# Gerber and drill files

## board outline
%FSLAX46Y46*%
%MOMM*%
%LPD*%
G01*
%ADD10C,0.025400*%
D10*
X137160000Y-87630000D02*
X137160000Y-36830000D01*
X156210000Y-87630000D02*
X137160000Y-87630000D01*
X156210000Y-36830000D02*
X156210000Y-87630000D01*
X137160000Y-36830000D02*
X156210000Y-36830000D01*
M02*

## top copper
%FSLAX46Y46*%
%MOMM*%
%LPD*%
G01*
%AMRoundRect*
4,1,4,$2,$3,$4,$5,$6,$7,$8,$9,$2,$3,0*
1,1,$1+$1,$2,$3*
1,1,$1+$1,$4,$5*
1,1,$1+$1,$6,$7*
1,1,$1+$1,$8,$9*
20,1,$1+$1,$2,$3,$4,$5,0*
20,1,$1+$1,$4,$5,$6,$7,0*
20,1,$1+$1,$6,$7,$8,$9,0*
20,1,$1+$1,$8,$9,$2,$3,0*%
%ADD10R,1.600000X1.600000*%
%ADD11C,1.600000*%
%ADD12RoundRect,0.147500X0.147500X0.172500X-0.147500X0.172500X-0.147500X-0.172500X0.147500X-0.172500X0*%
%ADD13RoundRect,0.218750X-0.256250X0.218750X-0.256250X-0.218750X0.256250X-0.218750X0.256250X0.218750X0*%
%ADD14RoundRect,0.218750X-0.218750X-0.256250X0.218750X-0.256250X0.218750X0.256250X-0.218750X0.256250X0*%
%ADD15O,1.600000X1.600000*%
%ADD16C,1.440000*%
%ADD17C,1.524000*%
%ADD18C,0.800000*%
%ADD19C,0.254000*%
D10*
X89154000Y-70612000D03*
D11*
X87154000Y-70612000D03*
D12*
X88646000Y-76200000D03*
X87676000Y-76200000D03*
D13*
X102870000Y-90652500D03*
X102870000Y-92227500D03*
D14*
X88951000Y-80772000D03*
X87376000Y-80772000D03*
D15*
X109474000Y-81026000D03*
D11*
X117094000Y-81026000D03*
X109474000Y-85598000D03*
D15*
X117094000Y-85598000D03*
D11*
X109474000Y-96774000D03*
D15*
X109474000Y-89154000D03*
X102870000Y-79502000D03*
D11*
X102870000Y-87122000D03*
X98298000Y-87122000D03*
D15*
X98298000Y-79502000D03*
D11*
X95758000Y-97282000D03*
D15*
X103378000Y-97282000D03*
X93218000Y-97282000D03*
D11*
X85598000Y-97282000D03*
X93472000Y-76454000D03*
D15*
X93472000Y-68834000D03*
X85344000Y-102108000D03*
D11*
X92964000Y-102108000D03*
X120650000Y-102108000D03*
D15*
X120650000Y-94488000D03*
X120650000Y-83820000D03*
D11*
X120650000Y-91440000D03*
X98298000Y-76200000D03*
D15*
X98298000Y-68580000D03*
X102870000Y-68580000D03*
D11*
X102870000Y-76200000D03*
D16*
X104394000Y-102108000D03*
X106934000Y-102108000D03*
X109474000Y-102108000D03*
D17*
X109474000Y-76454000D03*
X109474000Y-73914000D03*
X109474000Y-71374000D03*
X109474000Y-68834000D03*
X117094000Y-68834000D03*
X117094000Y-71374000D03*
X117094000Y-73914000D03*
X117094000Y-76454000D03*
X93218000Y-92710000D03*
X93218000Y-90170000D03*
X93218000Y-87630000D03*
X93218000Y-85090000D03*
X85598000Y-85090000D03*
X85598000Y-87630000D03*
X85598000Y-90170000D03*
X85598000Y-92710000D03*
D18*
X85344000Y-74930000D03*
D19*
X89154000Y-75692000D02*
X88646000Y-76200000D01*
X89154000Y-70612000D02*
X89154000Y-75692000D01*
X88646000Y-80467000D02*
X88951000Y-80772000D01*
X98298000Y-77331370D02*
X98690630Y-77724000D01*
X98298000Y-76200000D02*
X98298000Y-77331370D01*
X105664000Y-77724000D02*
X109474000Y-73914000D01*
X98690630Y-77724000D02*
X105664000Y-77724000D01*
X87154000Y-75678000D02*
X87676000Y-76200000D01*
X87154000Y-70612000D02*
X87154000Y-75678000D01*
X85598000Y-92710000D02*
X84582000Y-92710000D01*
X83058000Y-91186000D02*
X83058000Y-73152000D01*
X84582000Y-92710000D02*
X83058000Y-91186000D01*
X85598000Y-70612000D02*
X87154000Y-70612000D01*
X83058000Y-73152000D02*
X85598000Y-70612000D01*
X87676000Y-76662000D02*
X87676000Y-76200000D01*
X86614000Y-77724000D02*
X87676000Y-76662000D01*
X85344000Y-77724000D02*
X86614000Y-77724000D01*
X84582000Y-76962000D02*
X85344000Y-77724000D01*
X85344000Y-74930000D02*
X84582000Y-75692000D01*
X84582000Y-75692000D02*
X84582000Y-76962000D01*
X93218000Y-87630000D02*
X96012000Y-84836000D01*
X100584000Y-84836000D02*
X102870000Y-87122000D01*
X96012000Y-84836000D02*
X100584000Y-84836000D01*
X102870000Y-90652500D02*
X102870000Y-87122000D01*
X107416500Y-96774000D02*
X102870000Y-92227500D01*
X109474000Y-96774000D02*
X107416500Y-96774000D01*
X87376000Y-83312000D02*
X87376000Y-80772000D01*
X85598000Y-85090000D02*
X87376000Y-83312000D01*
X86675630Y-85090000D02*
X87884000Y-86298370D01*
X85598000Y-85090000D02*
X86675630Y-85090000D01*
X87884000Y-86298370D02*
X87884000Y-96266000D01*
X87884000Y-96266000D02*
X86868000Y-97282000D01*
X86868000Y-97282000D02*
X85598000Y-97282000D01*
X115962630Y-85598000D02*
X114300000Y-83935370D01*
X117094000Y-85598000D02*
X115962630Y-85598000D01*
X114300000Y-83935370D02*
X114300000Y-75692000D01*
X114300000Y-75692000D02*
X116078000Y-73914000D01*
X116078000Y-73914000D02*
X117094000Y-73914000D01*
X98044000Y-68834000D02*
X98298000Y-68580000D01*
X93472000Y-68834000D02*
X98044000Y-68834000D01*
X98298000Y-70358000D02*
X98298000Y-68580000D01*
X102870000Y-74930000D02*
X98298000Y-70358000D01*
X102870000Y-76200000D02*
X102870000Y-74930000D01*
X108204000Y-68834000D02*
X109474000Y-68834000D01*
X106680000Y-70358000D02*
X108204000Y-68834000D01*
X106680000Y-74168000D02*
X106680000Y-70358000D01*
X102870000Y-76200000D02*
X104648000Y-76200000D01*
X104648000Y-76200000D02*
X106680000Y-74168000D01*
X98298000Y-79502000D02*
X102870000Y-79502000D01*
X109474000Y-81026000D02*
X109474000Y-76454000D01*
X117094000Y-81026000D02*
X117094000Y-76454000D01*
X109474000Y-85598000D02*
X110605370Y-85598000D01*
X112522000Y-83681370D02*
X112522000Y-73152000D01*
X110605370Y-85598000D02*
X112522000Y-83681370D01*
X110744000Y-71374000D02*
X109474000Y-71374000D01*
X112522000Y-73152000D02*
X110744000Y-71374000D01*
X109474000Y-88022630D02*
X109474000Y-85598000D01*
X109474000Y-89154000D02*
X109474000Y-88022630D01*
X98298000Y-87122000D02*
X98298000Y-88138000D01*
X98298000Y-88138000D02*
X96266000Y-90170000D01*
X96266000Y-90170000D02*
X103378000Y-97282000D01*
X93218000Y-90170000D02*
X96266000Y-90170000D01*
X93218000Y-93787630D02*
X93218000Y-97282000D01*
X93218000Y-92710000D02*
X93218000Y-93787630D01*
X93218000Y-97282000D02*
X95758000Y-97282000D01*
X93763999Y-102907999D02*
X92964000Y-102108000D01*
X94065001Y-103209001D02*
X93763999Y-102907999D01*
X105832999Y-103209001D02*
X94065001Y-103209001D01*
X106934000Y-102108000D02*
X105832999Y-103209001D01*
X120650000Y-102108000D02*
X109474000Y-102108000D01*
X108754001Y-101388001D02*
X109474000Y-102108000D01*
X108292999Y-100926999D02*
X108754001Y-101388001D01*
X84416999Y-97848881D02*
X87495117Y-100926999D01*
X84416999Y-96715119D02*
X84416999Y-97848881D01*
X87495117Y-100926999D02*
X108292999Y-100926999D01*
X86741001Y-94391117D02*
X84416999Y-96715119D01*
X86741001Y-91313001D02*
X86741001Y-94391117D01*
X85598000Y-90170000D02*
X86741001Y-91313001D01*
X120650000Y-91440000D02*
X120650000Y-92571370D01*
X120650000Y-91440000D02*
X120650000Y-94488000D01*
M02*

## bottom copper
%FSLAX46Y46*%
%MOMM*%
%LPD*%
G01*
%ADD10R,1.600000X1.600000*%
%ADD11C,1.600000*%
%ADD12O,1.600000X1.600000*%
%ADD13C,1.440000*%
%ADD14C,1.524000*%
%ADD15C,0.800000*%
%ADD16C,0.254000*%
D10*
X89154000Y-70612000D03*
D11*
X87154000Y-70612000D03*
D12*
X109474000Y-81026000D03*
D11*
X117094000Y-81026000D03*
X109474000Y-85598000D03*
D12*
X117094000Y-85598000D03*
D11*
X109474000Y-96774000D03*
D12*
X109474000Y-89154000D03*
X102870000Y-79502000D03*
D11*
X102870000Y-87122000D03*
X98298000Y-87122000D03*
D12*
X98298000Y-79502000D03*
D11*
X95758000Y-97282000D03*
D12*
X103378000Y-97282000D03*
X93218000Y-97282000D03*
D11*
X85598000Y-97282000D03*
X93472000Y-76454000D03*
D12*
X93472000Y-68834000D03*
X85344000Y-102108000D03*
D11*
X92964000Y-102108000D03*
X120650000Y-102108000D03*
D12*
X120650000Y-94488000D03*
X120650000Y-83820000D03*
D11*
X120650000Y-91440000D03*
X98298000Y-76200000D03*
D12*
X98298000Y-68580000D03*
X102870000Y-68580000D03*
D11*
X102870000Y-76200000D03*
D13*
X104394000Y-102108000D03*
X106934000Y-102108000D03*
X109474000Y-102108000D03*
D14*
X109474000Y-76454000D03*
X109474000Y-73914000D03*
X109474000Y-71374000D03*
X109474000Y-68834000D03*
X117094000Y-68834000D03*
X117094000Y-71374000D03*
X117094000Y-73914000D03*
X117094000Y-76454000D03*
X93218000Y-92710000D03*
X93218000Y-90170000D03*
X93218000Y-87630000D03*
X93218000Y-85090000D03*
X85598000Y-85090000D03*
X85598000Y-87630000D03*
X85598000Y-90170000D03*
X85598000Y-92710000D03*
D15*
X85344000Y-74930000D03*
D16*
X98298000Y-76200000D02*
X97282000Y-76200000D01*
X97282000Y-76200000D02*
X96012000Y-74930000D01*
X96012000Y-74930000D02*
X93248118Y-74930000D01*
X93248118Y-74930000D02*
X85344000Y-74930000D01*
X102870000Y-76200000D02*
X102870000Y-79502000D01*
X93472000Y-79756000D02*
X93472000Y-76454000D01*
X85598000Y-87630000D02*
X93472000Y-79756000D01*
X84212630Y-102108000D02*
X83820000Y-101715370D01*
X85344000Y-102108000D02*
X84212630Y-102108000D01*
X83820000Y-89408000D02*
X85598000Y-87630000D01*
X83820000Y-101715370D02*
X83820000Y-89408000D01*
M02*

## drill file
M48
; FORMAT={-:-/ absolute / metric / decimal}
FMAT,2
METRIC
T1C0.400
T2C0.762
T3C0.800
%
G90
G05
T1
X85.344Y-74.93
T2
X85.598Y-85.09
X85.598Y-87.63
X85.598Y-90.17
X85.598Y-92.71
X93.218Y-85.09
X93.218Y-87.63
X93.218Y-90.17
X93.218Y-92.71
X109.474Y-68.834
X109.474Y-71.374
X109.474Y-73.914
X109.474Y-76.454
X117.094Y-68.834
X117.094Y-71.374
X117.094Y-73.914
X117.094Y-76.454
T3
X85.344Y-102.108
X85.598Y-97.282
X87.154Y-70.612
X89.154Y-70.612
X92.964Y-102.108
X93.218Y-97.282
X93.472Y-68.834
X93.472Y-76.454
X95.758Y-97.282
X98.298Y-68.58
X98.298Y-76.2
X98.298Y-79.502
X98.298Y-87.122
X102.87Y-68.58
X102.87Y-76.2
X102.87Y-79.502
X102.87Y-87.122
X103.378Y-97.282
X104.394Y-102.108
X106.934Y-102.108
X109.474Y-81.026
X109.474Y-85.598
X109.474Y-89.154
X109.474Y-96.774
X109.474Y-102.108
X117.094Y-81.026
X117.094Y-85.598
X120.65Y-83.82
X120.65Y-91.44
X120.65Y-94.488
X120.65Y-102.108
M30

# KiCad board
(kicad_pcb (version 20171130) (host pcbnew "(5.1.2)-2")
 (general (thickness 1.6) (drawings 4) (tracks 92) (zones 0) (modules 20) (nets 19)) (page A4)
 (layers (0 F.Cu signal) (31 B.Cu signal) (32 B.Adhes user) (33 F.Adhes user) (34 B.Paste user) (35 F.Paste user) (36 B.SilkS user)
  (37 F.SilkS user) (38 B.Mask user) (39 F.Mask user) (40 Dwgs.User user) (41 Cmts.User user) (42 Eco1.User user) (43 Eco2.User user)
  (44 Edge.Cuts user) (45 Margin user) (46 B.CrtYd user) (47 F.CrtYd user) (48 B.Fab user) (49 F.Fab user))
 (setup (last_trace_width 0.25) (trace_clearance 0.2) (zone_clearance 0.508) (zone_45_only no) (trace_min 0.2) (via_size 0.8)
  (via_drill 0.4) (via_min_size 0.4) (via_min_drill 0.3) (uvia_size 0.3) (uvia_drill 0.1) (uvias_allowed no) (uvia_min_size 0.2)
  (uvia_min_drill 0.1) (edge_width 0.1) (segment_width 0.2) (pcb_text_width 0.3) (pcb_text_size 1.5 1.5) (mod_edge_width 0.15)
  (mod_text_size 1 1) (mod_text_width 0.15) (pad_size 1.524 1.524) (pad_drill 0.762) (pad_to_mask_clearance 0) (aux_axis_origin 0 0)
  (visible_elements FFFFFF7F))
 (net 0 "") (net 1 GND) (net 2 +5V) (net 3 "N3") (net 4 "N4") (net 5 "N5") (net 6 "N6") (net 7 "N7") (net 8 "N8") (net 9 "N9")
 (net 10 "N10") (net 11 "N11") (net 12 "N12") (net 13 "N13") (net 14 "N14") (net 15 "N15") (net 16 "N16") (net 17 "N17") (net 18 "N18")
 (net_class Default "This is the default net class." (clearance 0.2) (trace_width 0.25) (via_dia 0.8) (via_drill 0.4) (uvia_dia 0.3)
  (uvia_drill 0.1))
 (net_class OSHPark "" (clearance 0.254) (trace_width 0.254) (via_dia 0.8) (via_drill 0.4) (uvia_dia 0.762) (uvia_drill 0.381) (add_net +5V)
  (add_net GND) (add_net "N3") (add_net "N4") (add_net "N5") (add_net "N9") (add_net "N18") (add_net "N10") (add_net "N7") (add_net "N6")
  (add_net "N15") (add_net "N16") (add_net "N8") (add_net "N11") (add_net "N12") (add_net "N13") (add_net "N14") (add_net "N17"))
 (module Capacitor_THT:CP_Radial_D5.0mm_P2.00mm (layer F.Cu) (at 89.154 70.612 180)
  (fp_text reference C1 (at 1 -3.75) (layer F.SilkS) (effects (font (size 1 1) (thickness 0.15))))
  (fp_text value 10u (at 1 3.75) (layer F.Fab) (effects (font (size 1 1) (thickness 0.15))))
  (pad 1 thru_hole rect (at 0 0 180) (size 1.6 1.6) (drill 0.8) (layers *.Cu *.Mask) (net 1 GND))
  (pad 2 thru_hole circle (at 2 0 180) (size 1.6 1.6) (drill 0.8) (layers *.Cu *.Mask) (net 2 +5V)))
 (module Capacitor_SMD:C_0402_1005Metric (layer F.Cu) (at 88.161 76.2 180)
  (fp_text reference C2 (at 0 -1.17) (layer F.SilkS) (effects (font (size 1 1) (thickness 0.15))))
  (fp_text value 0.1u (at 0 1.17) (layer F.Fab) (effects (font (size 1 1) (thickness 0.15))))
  (pad 1 smd roundrect (at -0.485 0 180) (size 0.59 0.64) (layers F.Cu F.Paste F.Mask) (roundrect_rratio 0.25) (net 1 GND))
  (pad 2 smd roundrect (at 0.485 0 180) (size 0.59 0.64) (layers F.Cu F.Paste F.Mask) (roundrect_rratio 0.25) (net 2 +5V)))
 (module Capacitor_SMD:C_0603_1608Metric (layer F.Cu) (at 102.87 91.44 270)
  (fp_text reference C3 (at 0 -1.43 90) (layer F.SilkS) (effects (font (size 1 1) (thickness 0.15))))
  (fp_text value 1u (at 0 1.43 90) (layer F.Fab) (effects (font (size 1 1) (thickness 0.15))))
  (pad 1 smd roundrect (at -0.7875 0 270) (size 0.875 0.95) (layers F.Cu F.Paste F.Mask) (roundrect_rratio 0.25) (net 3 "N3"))
  (pad 2 smd roundrect (at 0.7875 0 270) (size 0.875 0.95) (layers F.Cu F.Paste F.Mask) (roundrect_rratio 0.25) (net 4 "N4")))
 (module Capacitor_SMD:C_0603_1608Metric (layer F.Cu) (at 88.1635 80.772)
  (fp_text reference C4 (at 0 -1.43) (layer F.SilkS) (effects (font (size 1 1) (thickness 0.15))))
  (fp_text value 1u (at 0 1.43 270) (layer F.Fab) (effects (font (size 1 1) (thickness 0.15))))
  (pad 2 smd roundrect (at 0.7875 0) (size 0.875 0.95) (layers F.Cu F.Paste F.Mask) (roundrect_rratio 0.25) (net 1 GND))
  (pad 1 smd roundrect (at -0.7875 0) (size 0.875 0.95) (layers F.Cu F.Paste F.Mask) (roundrect_rratio 0.25) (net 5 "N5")))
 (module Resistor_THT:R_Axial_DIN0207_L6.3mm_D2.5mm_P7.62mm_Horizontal (layer F.Cu) (at 117.094 81.026 180)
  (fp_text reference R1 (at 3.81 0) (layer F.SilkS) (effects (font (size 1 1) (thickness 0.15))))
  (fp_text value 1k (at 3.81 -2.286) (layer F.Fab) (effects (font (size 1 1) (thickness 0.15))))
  (pad 2 thru_hole oval (at 7.62 0 180) (size 1.6 1.6) (drill 0.8) (layers *.Cu *.Mask) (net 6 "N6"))
  (pad 1 thru_hole circle (at 0 0 180) (size 1.6 1.6) (drill 0.8) (layers *.Cu *.Mask) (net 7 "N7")))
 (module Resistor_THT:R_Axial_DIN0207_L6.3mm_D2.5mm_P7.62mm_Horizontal (layer F.Cu) (at 109.474 85.598)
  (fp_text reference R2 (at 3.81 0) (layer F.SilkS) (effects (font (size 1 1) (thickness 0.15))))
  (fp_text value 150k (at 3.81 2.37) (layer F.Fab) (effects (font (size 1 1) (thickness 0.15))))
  (pad 1 thru_hole circle (at 0 0) (size 1.6 1.6) (drill 0.8) (layers *.Cu *.Mask) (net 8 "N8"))
  (pad 2 thru_hole oval (at 7.62 0) (size 1.6 1.6) (drill 0.8) (layers *.Cu *.Mask) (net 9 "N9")))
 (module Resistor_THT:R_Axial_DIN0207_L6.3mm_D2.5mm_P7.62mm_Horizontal (layer F.Cu) (at 109.474 96.774 90)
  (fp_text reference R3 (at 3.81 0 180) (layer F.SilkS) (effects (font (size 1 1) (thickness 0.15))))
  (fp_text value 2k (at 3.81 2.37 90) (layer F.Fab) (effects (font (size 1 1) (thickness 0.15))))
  (pad 1 thru_hole circle (at 0 0 90) (size 1.6 1.6) (drill 0.8) (layers *.Cu *.Mask) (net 4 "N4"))
  (pad 2 thru_hole oval (at 7.62 0 90) (size 1.6 1.6) (drill 0.8) (layers *.Cu *.Mask) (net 8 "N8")))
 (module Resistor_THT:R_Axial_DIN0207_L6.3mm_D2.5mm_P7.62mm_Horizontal (layer F.Cu) (at 102.87 87.122 90)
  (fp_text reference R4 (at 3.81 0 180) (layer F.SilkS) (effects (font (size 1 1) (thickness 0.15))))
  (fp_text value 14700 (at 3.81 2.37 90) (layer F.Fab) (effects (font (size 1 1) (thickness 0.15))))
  (pad 2 thru_hole oval (at 7.62 0 90) (size 1.6 1.6) (drill 0.8) (layers *.Cu *.Mask) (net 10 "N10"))
  (pad 1 thru_hole circle (at 0 0 90) (size 1.6 1.6) (drill 0.8) (layers *.Cu *.Mask) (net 3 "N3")))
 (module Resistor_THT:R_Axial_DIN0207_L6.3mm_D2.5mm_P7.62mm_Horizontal (layer F.Cu) (at 98.298 87.122 90)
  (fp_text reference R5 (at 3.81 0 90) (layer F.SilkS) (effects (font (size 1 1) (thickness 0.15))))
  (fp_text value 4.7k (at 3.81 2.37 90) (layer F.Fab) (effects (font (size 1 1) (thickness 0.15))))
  (pad 1 thru_hole circle (at 0 0 90) (size 1.6 1.6) (drill 0.8) (layers *.Cu *.Mask) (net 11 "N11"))
  (pad 2 thru_hole oval (at 7.62 0 90) (size 1.6 1.6) (drill 0.8) (layers *.Cu *.Mask) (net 10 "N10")))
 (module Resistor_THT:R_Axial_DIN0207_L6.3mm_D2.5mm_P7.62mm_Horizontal (layer F.Cu) (at 95.758 97.282)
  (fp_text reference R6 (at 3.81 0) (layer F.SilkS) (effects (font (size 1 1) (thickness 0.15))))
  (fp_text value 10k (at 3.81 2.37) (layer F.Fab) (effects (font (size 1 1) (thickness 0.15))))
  (pad 1 thru_hole circle (at 0 0) (size 1.6 1.6) (drill 0.8) (layers *.Cu *.Mask) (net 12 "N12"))
  (pad 2 thru_hole oval (at 7.62 0) (size 1.6 1.6) (drill 0.8) (layers *.Cu *.Mask) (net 11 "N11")))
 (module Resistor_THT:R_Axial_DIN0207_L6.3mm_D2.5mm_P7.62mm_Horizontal (layer F.Cu) (at 85.598 97.282)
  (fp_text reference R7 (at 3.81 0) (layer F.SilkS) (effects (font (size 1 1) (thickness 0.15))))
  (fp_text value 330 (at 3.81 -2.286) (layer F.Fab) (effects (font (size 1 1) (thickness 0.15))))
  (pad 2 thru_hole oval (at 7.62 0) (size 1.6 1.6) (drill 0.8) (layers *.Cu *.Mask) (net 12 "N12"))
  (pad 1 thru_hole circle (at 0 0) (size 1.6 1.6) (drill 0.8) (layers *.Cu *.Mask) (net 5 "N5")))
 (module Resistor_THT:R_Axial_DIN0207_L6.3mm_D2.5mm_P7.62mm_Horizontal (layer F.Cu) (at 93.472 76.454 90)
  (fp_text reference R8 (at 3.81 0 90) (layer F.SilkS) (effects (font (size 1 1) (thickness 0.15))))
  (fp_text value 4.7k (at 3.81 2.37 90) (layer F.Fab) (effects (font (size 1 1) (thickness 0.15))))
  (pad 1 thru_hole circle (at 0 0 90) (size 1.6 1.6) (drill 0.8) (layers *.Cu *.Mask) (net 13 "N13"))
  (pad 2 thru_hole oval (at 7.62 0 90) (size 1.6 1.6) (drill 0.8) (layers *.Cu *.Mask) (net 10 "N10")))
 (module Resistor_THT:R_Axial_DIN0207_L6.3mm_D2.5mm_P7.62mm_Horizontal (layer F.Cu) (at 92.964 102.108 180)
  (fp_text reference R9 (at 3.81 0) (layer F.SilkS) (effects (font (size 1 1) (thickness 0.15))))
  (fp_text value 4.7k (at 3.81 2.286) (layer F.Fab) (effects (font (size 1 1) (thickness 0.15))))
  (pad 2 thru_hole oval (at 7.62 0 180) (size 1.6 1.6) (drill 0.8) (layers *.Cu *.Mask) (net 13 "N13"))
  (pad 1 thru_hole circle (at 0 0 180) (size 1.6 1.6) (drill 0.8) (layers *.Cu *.Mask) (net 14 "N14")))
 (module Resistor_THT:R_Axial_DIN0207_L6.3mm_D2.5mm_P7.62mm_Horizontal (layer F.Cu) (at 120.65 102.108 90)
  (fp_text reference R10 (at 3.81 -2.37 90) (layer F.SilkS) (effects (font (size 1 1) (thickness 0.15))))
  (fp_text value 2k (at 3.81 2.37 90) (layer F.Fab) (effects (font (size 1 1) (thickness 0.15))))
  (pad 1 thru_hole circle (at 0 0 90) (size 1.6 1.6) (drill 0.8) (layers *.Cu *.Mask) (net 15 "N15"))
  (pad 2 thru_hole oval (at 7.62 0 90) (size 1.6 1.6) (drill 0.8) (layers *.Cu *.Mask) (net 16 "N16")))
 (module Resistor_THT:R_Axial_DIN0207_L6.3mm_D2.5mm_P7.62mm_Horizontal (layer F.Cu) (at 120.65 91.44 90)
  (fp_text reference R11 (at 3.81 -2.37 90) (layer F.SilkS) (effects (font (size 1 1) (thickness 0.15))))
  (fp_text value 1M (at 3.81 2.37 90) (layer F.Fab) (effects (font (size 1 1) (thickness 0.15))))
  (pad 2 thru_hole oval (at 7.62 0 90) (size 1.6 1.6) (drill 0.8) (layers *.Cu *.Mask) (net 1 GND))
  (pad 1 thru_hole circle (at 0 0 90) (size 1.6 1.6) (drill 0.8) (layers *.Cu *.Mask) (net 16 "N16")))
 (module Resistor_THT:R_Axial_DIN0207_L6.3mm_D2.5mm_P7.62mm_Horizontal (layer F.Cu) (at 98.298 76.2 90)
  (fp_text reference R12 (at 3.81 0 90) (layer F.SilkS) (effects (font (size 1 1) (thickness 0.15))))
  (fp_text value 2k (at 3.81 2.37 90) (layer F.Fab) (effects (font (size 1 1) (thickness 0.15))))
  (pad 1 thru_hole circle (at 0 0 90) (size 1.6 1.6) (drill 0.8) (layers *.Cu *.Mask) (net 2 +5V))
  (pad 2 thru_hole oval (at 7.62 0 90) (size 1.6 1.6) (drill 0.8) (layers *.Cu *.Mask) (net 10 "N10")))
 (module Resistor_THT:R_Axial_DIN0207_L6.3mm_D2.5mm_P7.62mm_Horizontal (layer F.Cu) (at 102.87 76.2 90)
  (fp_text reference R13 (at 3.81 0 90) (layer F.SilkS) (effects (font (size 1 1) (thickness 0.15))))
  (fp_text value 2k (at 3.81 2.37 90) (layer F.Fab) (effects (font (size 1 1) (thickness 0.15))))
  (pad 2 thru_hole oval (at 7.62 0 90) (size 1.6 1.6) (drill 0.8) (layers *.Cu *.Mask) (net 1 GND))
  (pad 1 thru_hole circle (at 0 0 90) (size 1.6 1.6) (drill 0.8) (layers *.Cu *.Mask) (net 10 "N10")))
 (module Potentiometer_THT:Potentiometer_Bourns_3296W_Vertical (layer F.Cu) (at 104.394 102.108 180)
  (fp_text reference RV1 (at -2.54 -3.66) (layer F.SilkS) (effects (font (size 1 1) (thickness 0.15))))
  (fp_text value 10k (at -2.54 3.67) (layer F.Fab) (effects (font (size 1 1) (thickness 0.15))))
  (pad 1 thru_hole circle (at 0 0 180) (size 1.44 1.44) (drill 0.8) (layers *.Cu *.Mask) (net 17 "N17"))
  (pad 2 thru_hole circle (at -2.54 0 180) (size 1.44 1.44) (drill 0.8) (layers *.Cu *.Mask) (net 14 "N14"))
  (pad 3 thru_hole circle (at -5.08 0 180) (size 1.44 1.44) (drill 0.8) (layers *.Cu *.Mask) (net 15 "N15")))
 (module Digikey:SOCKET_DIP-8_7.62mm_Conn (layer F.Cu) (at 117.094 76.454 180)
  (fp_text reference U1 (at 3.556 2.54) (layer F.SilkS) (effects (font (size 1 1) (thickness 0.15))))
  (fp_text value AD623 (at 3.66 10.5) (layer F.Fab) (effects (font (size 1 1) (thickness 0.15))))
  (pad 8 thru_hole circle (at 7.62 0 180) (size 1.524 1.524) (drill 0.762) (layers *.Cu *.Mask) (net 6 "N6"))
  (pad 7 thru_hole circle (at 7.62 2.54 180) (size 1.524 1.524) (drill 0.762) (layers *.Cu *.Mask) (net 2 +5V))
  (pad 6 thru_hole circle (at 7.62 5.08 180) (size 1.524 1.524) (drill 0.762) (layers *.Cu *.Mask) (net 8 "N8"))
  (pad 5 thru_hole circle (at 7.62 7.62 180) (size 1.524 1.524) (drill 0.762) (layers *.Cu *.Mask) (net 10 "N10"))
  (pad 4 thru_hole circle (at 0 7.62 180) (size 1.524 1.524) (drill 0.762) (layers *.Cu *.Mask) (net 1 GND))
  (pad 3 thru_hole circle (at 0 5.08 180) (size 1.524 1.524) (drill 0.762) (layers *.Cu *.Mask) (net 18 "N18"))
  (pad 2 thru_hole circle (at 0 2.54 180) (size 1.524 1.524) (drill 0.762) (layers *.Cu *.Mask) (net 9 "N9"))
  (pad 1 thru_hole circle (at 0 0 180) (size 1.524 1.524) (drill 0.762) (layers *.Cu *.Mask) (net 7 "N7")))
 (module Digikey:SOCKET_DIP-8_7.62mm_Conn (layer F.Cu) (at 93.218 92.71 180)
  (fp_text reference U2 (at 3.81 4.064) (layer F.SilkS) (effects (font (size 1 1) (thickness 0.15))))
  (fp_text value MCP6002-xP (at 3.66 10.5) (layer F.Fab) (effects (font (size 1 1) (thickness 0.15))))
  (pad 1 thru_hole circle (at 0 0 180) (size 1.524 1.524) (drill 0.762) (layers *.Cu *.Mask) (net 12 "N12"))
  (pad 2 thru_hole circle (at 0 2.54 180) (size 1.524 1.524) (drill 0.762) (layers *.Cu *.Mask) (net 11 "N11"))
  (pad 3 thru_hole circle (at 0 5.08 180) (size 1.524 1.524) (drill 0.762) (layers *.Cu *.Mask) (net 3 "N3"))
  (pad 4 thru_hole circle (at 0 7.62 180) (size 1.524 1.524) (drill 0.762) (layers *.Cu *.Mask) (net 1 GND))
  (pad 5 thru_hole circle (at 7.62 7.62 180) (size 1.524 1.524) (drill 0.762) (layers *.Cu *.Mask) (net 5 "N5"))
  (pad 6 thru_hole circle (at 7.62 5.08 180) (size 1.524 1.524) (drill 0.762) (layers *.Cu *.Mask) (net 13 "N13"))
  (pad 7 thru_hole circle (at 7.62 2.54 180) (size 1.524 1.524) (drill 0.762) (layers *.Cu *.Mask) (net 15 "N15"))
  (pad 8 thru_hole circle (at 7.62 0 180) (size 1.524 1.524) (drill 0.762) (layers *.Cu *.Mask) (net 2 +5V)))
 (gr_line (start 137.16 87.63) (end 137.16 36.83) (layer Edge.Cuts) (width 0.0254))
 (gr_line (start 156.21 87.63) (end 137.16 87.63) (layer Edge.Cuts) (width 0.0254))
 (gr_line (start 156.21 36.83) (end 156.21 87.63) (layer Edge.Cuts) (width 0.0254))
 (gr_line (start 137.16 36.83) (end 156.21 36.83) (layer Edge.Cuts) (width 0.0254))
 (segment (start 89.154 75.692) (end 88.646 76.2) (width 0.254) (layer F.Cu) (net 1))
 (segment (start 89.154 70.612) (end 89.154 75.692) (width 0.254) (layer F.Cu) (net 1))
 (segment (start 88.646 80.467) (end 88.951 80.772) (width 0.254) (layer F.Cu) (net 1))
 (segment (start 98.298 77.33137) (end 98.69063 77.724) (width 0.254) (layer F.Cu) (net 2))
 (segment (start 98.298 76.2) (end 98.298 77.33137) (width 0.254) (layer F.Cu) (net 2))
 (segment (start 105.664 77.724) (end 109.474 73.914) (width 0.254) (layer F.Cu) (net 2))
 (segment (start 98.69063 77.724) (end 105.664 77.724) (width 0.254) (layer F.Cu) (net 2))
 (segment (start 87.154 75.678) (end 87.676 76.2) (width 0.254) (layer F.Cu) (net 2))
 (segment (start 87.154 70.612) (end 87.154 75.678) (width 0.254) (layer F.Cu) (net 2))
 (segment (start 85.598 92.71) (end 84.582 92.71) (width 0.254) (layer F.Cu) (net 2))
 (segment (start 83.058 91.186) (end 83.058 73.152) (width 0.254) (layer F.Cu) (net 2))
 (segment (start 84.582 92.71) (end 83.058 91.186) (width 0.254) (layer F.Cu) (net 2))
 (segment (start 85.598 70.612) (end 87.154 70.612) (width 0.254) (layer F.Cu) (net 2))
 (segment (start 83.058 73.152) (end 85.598 70.612) (width 0.254) (layer F.Cu) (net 2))
 (segment (start 98.298 76.2) (end 97.282 76.2) (width 0.254) (layer B.Cu) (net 2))
 (segment (start 97.282 76.2) (end 96.012 74.93) (width 0.254) (layer B.Cu) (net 2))
 (via (at 85.344 74.93) (size 0.8) (drill 0.4) (layers F.Cu B.Cu) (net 2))
 (segment (start 96.012 74.93) (end 93.248118 74.93) (width 0.254) (layer B.Cu) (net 2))
 (segment (start 93.248118 74.93) (end 85.344 74.93) (width 0.254) (layer B.Cu) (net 2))
 (segment (start 87.676 76.662) (end 87.676 76.2) (width 0.254) (layer F.Cu) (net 2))
 (segment (start 86.614 77.724) (end 87.676 76.662) (width 0.254) (layer F.Cu) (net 2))
 (segment (start 85.344 77.724) (end 86.614 77.724) (width 0.254) (layer F.Cu) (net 2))
 (segment (start 84.582 76.962) (end 85.344 77.724) (width 0.254) (layer F.Cu) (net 2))
 (segment (start 85.344 74.93) (end 84.582 75.692) (width 0.254) (layer F.Cu) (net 2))
 (segment (start 84.582 75.692) (end 84.582 76.962) (width 0.254) (layer F.Cu) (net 2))
 (segment (start 93.218 87.63) (end 96.012 84.836) (width 0.254) (layer F.Cu) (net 3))
 (segment (start 100.584 84.836) (end 102.87 87.122) (width 0.254) (layer F.Cu) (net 3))
 (segment (start 96.012 84.836) (end 100.584 84.836) (width 0.254) (layer F.Cu) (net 3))
 (segment (start 102.87 90.6525) (end 102.87 87.122) (width 0.254) (layer F.Cu) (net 3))
 (segment (start 107.4165 96.774) (end 102.87 92.2275) (width 0.254) (layer F.Cu) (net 4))
 (segment (start 109.474 96.774) (end 107.4165 96.774) (width 0.254) (layer F.Cu) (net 4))
 (segment (start 87.376 83.312) (end 87.376 80.772) (width 0.254) (layer F.Cu) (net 5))
 (segment (start 85.598 85.09) (end 87.376 83.312) (width 0.254) (layer F.Cu) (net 5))
 (segment (start 86.67563 85.09) (end 87.884 86.29837) (width 0.254) (layer F.Cu) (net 5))
 (segment (start 85.598 85.09) (end 86.67563 85.09) (width 0.254) (layer F.Cu) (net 5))
 (segment (start 87.884 86.29837) (end 87.884 96.266) (width 0.254) (layer F.Cu) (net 5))
 (segment (start 87.884 96.266) (end 86.868 97.282) (width 0.254) (layer F.Cu) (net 5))
 (segment (start 86.868 97.282) (end 85.598 97.282) (width 0.254) (layer F.Cu) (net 5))
 (segment (start 115.96263 85.598) (end 114.3 83.93537) (width 0.254) (layer F.Cu) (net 9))
 (segment (start 117.094 85.598) (end 115.96263 85.598) (width 0.254) (layer F.Cu) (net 9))
 (segment (start 114.3 83.93537) (end 114.3 75.692) (width 0.254) (layer F.Cu) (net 9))
 (segment (start 114.3 75.692) (end 116.078 73.914) (width 0.254) (layer F.Cu) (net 9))
 (segment (start 116.078 73.914) (end 117.094 73.914) (width 0.254) (layer F.Cu) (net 9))
 (segment (start 98.044 68.834) (end 98.298 68.58) (width 0.254) (layer F.Cu) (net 10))
 (segment (start 93.472 68.834) (end 98.044 68.834) (width 0.254) (layer F.Cu) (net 10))
 (segment (start 98.298 70.358) (end 98.298 68.58) (width 0.254) (layer F.Cu) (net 10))
 (segment (start 102.87 74.93) (end 98.298 70.358) (width 0.254) (layer F.Cu) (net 10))
 (segment (start 102.87 76.2) (end 102.87 74.93) (width 0.254) (layer F.Cu) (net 10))
 (segment (start 108.204 68.834) (end 109.474 68.834) (width 0.254) (layer F.Cu) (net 10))
 (segment (start 106.68 70.358) (end 108.204 68.834) (width 0.254) (layer F.Cu) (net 10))
 (segment (start 106.68 74.168) (end 106.68 70.358) (width 0.254) (layer F.Cu) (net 10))
 (segment (start 102.87 76.2) (end 104.648 76.2) (width 0.254) (layer F.Cu) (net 10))
 (segment (start 104.648 76.2) (end 106.68 74.168) (width 0.254) (layer F.Cu) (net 10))
 (segment (start 98.298 79.502) (end 102.87 79.502) (width 0.254) (layer F.Cu) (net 10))
 (segment (start 102.87 76.2) (end 102.87 79.502) (width 0.254) (layer B.Cu) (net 10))
 (segment (start 109.474 81.026) (end 109.474 76.454) (width 0.254) (layer F.Cu) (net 6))
 (segment (start 117.094 81.026) (end 117.094 76.454) (width 0.254) (layer F.Cu) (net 7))
 (segment (start 109.474 85.598) (end 110.60537 85.598) (width 0.254) (layer F.Cu) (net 8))
 (segment (start 112.522 83.68137) (end 112.522 73.152) (width 0.254) (layer F.Cu) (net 8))
 (segment (start 110.60537 85.598) (end 112.522 83.68137) (width 0.254) (layer F.Cu) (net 8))
 (segment (start 110.744 71.374) (end 109.474 71.374) (width 0.254) (layer F.Cu) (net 8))
 (segment (start 112.522 73.152) (end 110.744 71.374) (width 0.254) (layer F.Cu) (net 8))
 (segment (start 109.474 88.02263) (end 109.474 85.598) (width 0.254) (layer F.Cu) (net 8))
 (segment (start 109.474 89.154) (end 109.474 88.02263) (width 0.254) (layer F.Cu) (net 8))
 (segment (start 98.298 87.122) (end 98.298 88.138) (width 0.254) (layer F.Cu) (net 11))
 (segment (start 98.298 88.138) (end 96.266 90.17) (width 0.254) (layer F.Cu) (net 11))
 (segment (start 96.266 90.17) (end 103.378 97.282) (width 0.254) (layer F.Cu) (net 11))
 (segment (start 93.218 90.17) (end 96.266 90.17) (width 0.254) (layer F.Cu) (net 11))
 (segment (start 93.218 93.78763) (end 93.218 97.282) (width 0.254) (layer F.Cu) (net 12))
 (segment (start 93.218 92.71) (end 93.218 93.78763) (width 0.254) (layer F.Cu) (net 12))
 (segment (start 93.218 97.282) (end 95.758 97.282) (width 0.254) (layer F.Cu) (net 12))
 (segment (start 93.472 79.756) (end 93.472 76.454) (width 0.254) (layer B.Cu) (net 13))
 (segment (start 85.598 87.63) (end 93.472 79.756) (width 0.254) (layer B.Cu) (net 13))
 (segment (start 84.21263 102.108) (end 83.82 101.71537) (width 0.254) (layer B.Cu) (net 13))
 (segment (start 85.344 102.108) (end 84.21263 102.108) (width 0.254) (layer B.Cu) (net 13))
 (segment (start 83.82 89.408) (end 85.598 87.63) (width 0.254) (layer B.Cu) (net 13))
 (segment (start 83.82 101.71537) (end 83.82 89.408) (width 0.254) (layer B.Cu) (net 13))
 (segment (start 93.763999 102.907999) (end 92.964 102.108) (width 0.254) (layer F.Cu) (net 14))
 (segment (start 94.065001 103.209001) (end 93.763999 102.907999) (width 0.254) (layer F.Cu) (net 14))
 (segment (start 105.832999 103.209001) (end 94.065001 103.209001) (width 0.254) (layer F.Cu) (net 14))
 (segment (start 106.934 102.108) (end 105.832999 103.209001) (width 0.254) (layer F.Cu) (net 14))
 (segment (start 120.65 102.108) (end 109.474 102.108) (width 0.254) (layer F.Cu) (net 15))
 (segment (start 108.754001 101.388001) (end 109.474 102.108) (width 0.254) (layer F.Cu) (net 15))
 (segment (start 108.292999 100.926999) (end 108.754001 101.388001) (width 0.254) (layer F.Cu) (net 15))
 (segment (start 84.416999 97.848881) (end 87.495117 100.926999) (width 0.254) (layer F.Cu) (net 15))
 (segment (start 84.416999 96.715119) (end 84.416999 97.848881) (width 0.254) (layer F.Cu) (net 15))
 (segment (start 87.495117 100.926999) (end 108.292999 100.926999) (width 0.254) (layer F.Cu) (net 15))
 (segment (start 86.741001 94.391117) (end 84.416999 96.715119) (width 0.254) (layer F.Cu) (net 15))
 (segment (start 86.741001 91.313001) (end 86.741001 94.391117) (width 0.254) (layer F.Cu) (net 15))
 (segment (start 85.598 90.17) (end 86.741001 91.313001) (width 0.254) (layer F.Cu) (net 15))
 (segment (start 120.65 91.44) (end 120.65 92.57137) (width 0.254) (layer F.Cu) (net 16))
 (segment (start 120.65 91.44) (end 120.65 94.488) (width 0.254) (layer F.Cu) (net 16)))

